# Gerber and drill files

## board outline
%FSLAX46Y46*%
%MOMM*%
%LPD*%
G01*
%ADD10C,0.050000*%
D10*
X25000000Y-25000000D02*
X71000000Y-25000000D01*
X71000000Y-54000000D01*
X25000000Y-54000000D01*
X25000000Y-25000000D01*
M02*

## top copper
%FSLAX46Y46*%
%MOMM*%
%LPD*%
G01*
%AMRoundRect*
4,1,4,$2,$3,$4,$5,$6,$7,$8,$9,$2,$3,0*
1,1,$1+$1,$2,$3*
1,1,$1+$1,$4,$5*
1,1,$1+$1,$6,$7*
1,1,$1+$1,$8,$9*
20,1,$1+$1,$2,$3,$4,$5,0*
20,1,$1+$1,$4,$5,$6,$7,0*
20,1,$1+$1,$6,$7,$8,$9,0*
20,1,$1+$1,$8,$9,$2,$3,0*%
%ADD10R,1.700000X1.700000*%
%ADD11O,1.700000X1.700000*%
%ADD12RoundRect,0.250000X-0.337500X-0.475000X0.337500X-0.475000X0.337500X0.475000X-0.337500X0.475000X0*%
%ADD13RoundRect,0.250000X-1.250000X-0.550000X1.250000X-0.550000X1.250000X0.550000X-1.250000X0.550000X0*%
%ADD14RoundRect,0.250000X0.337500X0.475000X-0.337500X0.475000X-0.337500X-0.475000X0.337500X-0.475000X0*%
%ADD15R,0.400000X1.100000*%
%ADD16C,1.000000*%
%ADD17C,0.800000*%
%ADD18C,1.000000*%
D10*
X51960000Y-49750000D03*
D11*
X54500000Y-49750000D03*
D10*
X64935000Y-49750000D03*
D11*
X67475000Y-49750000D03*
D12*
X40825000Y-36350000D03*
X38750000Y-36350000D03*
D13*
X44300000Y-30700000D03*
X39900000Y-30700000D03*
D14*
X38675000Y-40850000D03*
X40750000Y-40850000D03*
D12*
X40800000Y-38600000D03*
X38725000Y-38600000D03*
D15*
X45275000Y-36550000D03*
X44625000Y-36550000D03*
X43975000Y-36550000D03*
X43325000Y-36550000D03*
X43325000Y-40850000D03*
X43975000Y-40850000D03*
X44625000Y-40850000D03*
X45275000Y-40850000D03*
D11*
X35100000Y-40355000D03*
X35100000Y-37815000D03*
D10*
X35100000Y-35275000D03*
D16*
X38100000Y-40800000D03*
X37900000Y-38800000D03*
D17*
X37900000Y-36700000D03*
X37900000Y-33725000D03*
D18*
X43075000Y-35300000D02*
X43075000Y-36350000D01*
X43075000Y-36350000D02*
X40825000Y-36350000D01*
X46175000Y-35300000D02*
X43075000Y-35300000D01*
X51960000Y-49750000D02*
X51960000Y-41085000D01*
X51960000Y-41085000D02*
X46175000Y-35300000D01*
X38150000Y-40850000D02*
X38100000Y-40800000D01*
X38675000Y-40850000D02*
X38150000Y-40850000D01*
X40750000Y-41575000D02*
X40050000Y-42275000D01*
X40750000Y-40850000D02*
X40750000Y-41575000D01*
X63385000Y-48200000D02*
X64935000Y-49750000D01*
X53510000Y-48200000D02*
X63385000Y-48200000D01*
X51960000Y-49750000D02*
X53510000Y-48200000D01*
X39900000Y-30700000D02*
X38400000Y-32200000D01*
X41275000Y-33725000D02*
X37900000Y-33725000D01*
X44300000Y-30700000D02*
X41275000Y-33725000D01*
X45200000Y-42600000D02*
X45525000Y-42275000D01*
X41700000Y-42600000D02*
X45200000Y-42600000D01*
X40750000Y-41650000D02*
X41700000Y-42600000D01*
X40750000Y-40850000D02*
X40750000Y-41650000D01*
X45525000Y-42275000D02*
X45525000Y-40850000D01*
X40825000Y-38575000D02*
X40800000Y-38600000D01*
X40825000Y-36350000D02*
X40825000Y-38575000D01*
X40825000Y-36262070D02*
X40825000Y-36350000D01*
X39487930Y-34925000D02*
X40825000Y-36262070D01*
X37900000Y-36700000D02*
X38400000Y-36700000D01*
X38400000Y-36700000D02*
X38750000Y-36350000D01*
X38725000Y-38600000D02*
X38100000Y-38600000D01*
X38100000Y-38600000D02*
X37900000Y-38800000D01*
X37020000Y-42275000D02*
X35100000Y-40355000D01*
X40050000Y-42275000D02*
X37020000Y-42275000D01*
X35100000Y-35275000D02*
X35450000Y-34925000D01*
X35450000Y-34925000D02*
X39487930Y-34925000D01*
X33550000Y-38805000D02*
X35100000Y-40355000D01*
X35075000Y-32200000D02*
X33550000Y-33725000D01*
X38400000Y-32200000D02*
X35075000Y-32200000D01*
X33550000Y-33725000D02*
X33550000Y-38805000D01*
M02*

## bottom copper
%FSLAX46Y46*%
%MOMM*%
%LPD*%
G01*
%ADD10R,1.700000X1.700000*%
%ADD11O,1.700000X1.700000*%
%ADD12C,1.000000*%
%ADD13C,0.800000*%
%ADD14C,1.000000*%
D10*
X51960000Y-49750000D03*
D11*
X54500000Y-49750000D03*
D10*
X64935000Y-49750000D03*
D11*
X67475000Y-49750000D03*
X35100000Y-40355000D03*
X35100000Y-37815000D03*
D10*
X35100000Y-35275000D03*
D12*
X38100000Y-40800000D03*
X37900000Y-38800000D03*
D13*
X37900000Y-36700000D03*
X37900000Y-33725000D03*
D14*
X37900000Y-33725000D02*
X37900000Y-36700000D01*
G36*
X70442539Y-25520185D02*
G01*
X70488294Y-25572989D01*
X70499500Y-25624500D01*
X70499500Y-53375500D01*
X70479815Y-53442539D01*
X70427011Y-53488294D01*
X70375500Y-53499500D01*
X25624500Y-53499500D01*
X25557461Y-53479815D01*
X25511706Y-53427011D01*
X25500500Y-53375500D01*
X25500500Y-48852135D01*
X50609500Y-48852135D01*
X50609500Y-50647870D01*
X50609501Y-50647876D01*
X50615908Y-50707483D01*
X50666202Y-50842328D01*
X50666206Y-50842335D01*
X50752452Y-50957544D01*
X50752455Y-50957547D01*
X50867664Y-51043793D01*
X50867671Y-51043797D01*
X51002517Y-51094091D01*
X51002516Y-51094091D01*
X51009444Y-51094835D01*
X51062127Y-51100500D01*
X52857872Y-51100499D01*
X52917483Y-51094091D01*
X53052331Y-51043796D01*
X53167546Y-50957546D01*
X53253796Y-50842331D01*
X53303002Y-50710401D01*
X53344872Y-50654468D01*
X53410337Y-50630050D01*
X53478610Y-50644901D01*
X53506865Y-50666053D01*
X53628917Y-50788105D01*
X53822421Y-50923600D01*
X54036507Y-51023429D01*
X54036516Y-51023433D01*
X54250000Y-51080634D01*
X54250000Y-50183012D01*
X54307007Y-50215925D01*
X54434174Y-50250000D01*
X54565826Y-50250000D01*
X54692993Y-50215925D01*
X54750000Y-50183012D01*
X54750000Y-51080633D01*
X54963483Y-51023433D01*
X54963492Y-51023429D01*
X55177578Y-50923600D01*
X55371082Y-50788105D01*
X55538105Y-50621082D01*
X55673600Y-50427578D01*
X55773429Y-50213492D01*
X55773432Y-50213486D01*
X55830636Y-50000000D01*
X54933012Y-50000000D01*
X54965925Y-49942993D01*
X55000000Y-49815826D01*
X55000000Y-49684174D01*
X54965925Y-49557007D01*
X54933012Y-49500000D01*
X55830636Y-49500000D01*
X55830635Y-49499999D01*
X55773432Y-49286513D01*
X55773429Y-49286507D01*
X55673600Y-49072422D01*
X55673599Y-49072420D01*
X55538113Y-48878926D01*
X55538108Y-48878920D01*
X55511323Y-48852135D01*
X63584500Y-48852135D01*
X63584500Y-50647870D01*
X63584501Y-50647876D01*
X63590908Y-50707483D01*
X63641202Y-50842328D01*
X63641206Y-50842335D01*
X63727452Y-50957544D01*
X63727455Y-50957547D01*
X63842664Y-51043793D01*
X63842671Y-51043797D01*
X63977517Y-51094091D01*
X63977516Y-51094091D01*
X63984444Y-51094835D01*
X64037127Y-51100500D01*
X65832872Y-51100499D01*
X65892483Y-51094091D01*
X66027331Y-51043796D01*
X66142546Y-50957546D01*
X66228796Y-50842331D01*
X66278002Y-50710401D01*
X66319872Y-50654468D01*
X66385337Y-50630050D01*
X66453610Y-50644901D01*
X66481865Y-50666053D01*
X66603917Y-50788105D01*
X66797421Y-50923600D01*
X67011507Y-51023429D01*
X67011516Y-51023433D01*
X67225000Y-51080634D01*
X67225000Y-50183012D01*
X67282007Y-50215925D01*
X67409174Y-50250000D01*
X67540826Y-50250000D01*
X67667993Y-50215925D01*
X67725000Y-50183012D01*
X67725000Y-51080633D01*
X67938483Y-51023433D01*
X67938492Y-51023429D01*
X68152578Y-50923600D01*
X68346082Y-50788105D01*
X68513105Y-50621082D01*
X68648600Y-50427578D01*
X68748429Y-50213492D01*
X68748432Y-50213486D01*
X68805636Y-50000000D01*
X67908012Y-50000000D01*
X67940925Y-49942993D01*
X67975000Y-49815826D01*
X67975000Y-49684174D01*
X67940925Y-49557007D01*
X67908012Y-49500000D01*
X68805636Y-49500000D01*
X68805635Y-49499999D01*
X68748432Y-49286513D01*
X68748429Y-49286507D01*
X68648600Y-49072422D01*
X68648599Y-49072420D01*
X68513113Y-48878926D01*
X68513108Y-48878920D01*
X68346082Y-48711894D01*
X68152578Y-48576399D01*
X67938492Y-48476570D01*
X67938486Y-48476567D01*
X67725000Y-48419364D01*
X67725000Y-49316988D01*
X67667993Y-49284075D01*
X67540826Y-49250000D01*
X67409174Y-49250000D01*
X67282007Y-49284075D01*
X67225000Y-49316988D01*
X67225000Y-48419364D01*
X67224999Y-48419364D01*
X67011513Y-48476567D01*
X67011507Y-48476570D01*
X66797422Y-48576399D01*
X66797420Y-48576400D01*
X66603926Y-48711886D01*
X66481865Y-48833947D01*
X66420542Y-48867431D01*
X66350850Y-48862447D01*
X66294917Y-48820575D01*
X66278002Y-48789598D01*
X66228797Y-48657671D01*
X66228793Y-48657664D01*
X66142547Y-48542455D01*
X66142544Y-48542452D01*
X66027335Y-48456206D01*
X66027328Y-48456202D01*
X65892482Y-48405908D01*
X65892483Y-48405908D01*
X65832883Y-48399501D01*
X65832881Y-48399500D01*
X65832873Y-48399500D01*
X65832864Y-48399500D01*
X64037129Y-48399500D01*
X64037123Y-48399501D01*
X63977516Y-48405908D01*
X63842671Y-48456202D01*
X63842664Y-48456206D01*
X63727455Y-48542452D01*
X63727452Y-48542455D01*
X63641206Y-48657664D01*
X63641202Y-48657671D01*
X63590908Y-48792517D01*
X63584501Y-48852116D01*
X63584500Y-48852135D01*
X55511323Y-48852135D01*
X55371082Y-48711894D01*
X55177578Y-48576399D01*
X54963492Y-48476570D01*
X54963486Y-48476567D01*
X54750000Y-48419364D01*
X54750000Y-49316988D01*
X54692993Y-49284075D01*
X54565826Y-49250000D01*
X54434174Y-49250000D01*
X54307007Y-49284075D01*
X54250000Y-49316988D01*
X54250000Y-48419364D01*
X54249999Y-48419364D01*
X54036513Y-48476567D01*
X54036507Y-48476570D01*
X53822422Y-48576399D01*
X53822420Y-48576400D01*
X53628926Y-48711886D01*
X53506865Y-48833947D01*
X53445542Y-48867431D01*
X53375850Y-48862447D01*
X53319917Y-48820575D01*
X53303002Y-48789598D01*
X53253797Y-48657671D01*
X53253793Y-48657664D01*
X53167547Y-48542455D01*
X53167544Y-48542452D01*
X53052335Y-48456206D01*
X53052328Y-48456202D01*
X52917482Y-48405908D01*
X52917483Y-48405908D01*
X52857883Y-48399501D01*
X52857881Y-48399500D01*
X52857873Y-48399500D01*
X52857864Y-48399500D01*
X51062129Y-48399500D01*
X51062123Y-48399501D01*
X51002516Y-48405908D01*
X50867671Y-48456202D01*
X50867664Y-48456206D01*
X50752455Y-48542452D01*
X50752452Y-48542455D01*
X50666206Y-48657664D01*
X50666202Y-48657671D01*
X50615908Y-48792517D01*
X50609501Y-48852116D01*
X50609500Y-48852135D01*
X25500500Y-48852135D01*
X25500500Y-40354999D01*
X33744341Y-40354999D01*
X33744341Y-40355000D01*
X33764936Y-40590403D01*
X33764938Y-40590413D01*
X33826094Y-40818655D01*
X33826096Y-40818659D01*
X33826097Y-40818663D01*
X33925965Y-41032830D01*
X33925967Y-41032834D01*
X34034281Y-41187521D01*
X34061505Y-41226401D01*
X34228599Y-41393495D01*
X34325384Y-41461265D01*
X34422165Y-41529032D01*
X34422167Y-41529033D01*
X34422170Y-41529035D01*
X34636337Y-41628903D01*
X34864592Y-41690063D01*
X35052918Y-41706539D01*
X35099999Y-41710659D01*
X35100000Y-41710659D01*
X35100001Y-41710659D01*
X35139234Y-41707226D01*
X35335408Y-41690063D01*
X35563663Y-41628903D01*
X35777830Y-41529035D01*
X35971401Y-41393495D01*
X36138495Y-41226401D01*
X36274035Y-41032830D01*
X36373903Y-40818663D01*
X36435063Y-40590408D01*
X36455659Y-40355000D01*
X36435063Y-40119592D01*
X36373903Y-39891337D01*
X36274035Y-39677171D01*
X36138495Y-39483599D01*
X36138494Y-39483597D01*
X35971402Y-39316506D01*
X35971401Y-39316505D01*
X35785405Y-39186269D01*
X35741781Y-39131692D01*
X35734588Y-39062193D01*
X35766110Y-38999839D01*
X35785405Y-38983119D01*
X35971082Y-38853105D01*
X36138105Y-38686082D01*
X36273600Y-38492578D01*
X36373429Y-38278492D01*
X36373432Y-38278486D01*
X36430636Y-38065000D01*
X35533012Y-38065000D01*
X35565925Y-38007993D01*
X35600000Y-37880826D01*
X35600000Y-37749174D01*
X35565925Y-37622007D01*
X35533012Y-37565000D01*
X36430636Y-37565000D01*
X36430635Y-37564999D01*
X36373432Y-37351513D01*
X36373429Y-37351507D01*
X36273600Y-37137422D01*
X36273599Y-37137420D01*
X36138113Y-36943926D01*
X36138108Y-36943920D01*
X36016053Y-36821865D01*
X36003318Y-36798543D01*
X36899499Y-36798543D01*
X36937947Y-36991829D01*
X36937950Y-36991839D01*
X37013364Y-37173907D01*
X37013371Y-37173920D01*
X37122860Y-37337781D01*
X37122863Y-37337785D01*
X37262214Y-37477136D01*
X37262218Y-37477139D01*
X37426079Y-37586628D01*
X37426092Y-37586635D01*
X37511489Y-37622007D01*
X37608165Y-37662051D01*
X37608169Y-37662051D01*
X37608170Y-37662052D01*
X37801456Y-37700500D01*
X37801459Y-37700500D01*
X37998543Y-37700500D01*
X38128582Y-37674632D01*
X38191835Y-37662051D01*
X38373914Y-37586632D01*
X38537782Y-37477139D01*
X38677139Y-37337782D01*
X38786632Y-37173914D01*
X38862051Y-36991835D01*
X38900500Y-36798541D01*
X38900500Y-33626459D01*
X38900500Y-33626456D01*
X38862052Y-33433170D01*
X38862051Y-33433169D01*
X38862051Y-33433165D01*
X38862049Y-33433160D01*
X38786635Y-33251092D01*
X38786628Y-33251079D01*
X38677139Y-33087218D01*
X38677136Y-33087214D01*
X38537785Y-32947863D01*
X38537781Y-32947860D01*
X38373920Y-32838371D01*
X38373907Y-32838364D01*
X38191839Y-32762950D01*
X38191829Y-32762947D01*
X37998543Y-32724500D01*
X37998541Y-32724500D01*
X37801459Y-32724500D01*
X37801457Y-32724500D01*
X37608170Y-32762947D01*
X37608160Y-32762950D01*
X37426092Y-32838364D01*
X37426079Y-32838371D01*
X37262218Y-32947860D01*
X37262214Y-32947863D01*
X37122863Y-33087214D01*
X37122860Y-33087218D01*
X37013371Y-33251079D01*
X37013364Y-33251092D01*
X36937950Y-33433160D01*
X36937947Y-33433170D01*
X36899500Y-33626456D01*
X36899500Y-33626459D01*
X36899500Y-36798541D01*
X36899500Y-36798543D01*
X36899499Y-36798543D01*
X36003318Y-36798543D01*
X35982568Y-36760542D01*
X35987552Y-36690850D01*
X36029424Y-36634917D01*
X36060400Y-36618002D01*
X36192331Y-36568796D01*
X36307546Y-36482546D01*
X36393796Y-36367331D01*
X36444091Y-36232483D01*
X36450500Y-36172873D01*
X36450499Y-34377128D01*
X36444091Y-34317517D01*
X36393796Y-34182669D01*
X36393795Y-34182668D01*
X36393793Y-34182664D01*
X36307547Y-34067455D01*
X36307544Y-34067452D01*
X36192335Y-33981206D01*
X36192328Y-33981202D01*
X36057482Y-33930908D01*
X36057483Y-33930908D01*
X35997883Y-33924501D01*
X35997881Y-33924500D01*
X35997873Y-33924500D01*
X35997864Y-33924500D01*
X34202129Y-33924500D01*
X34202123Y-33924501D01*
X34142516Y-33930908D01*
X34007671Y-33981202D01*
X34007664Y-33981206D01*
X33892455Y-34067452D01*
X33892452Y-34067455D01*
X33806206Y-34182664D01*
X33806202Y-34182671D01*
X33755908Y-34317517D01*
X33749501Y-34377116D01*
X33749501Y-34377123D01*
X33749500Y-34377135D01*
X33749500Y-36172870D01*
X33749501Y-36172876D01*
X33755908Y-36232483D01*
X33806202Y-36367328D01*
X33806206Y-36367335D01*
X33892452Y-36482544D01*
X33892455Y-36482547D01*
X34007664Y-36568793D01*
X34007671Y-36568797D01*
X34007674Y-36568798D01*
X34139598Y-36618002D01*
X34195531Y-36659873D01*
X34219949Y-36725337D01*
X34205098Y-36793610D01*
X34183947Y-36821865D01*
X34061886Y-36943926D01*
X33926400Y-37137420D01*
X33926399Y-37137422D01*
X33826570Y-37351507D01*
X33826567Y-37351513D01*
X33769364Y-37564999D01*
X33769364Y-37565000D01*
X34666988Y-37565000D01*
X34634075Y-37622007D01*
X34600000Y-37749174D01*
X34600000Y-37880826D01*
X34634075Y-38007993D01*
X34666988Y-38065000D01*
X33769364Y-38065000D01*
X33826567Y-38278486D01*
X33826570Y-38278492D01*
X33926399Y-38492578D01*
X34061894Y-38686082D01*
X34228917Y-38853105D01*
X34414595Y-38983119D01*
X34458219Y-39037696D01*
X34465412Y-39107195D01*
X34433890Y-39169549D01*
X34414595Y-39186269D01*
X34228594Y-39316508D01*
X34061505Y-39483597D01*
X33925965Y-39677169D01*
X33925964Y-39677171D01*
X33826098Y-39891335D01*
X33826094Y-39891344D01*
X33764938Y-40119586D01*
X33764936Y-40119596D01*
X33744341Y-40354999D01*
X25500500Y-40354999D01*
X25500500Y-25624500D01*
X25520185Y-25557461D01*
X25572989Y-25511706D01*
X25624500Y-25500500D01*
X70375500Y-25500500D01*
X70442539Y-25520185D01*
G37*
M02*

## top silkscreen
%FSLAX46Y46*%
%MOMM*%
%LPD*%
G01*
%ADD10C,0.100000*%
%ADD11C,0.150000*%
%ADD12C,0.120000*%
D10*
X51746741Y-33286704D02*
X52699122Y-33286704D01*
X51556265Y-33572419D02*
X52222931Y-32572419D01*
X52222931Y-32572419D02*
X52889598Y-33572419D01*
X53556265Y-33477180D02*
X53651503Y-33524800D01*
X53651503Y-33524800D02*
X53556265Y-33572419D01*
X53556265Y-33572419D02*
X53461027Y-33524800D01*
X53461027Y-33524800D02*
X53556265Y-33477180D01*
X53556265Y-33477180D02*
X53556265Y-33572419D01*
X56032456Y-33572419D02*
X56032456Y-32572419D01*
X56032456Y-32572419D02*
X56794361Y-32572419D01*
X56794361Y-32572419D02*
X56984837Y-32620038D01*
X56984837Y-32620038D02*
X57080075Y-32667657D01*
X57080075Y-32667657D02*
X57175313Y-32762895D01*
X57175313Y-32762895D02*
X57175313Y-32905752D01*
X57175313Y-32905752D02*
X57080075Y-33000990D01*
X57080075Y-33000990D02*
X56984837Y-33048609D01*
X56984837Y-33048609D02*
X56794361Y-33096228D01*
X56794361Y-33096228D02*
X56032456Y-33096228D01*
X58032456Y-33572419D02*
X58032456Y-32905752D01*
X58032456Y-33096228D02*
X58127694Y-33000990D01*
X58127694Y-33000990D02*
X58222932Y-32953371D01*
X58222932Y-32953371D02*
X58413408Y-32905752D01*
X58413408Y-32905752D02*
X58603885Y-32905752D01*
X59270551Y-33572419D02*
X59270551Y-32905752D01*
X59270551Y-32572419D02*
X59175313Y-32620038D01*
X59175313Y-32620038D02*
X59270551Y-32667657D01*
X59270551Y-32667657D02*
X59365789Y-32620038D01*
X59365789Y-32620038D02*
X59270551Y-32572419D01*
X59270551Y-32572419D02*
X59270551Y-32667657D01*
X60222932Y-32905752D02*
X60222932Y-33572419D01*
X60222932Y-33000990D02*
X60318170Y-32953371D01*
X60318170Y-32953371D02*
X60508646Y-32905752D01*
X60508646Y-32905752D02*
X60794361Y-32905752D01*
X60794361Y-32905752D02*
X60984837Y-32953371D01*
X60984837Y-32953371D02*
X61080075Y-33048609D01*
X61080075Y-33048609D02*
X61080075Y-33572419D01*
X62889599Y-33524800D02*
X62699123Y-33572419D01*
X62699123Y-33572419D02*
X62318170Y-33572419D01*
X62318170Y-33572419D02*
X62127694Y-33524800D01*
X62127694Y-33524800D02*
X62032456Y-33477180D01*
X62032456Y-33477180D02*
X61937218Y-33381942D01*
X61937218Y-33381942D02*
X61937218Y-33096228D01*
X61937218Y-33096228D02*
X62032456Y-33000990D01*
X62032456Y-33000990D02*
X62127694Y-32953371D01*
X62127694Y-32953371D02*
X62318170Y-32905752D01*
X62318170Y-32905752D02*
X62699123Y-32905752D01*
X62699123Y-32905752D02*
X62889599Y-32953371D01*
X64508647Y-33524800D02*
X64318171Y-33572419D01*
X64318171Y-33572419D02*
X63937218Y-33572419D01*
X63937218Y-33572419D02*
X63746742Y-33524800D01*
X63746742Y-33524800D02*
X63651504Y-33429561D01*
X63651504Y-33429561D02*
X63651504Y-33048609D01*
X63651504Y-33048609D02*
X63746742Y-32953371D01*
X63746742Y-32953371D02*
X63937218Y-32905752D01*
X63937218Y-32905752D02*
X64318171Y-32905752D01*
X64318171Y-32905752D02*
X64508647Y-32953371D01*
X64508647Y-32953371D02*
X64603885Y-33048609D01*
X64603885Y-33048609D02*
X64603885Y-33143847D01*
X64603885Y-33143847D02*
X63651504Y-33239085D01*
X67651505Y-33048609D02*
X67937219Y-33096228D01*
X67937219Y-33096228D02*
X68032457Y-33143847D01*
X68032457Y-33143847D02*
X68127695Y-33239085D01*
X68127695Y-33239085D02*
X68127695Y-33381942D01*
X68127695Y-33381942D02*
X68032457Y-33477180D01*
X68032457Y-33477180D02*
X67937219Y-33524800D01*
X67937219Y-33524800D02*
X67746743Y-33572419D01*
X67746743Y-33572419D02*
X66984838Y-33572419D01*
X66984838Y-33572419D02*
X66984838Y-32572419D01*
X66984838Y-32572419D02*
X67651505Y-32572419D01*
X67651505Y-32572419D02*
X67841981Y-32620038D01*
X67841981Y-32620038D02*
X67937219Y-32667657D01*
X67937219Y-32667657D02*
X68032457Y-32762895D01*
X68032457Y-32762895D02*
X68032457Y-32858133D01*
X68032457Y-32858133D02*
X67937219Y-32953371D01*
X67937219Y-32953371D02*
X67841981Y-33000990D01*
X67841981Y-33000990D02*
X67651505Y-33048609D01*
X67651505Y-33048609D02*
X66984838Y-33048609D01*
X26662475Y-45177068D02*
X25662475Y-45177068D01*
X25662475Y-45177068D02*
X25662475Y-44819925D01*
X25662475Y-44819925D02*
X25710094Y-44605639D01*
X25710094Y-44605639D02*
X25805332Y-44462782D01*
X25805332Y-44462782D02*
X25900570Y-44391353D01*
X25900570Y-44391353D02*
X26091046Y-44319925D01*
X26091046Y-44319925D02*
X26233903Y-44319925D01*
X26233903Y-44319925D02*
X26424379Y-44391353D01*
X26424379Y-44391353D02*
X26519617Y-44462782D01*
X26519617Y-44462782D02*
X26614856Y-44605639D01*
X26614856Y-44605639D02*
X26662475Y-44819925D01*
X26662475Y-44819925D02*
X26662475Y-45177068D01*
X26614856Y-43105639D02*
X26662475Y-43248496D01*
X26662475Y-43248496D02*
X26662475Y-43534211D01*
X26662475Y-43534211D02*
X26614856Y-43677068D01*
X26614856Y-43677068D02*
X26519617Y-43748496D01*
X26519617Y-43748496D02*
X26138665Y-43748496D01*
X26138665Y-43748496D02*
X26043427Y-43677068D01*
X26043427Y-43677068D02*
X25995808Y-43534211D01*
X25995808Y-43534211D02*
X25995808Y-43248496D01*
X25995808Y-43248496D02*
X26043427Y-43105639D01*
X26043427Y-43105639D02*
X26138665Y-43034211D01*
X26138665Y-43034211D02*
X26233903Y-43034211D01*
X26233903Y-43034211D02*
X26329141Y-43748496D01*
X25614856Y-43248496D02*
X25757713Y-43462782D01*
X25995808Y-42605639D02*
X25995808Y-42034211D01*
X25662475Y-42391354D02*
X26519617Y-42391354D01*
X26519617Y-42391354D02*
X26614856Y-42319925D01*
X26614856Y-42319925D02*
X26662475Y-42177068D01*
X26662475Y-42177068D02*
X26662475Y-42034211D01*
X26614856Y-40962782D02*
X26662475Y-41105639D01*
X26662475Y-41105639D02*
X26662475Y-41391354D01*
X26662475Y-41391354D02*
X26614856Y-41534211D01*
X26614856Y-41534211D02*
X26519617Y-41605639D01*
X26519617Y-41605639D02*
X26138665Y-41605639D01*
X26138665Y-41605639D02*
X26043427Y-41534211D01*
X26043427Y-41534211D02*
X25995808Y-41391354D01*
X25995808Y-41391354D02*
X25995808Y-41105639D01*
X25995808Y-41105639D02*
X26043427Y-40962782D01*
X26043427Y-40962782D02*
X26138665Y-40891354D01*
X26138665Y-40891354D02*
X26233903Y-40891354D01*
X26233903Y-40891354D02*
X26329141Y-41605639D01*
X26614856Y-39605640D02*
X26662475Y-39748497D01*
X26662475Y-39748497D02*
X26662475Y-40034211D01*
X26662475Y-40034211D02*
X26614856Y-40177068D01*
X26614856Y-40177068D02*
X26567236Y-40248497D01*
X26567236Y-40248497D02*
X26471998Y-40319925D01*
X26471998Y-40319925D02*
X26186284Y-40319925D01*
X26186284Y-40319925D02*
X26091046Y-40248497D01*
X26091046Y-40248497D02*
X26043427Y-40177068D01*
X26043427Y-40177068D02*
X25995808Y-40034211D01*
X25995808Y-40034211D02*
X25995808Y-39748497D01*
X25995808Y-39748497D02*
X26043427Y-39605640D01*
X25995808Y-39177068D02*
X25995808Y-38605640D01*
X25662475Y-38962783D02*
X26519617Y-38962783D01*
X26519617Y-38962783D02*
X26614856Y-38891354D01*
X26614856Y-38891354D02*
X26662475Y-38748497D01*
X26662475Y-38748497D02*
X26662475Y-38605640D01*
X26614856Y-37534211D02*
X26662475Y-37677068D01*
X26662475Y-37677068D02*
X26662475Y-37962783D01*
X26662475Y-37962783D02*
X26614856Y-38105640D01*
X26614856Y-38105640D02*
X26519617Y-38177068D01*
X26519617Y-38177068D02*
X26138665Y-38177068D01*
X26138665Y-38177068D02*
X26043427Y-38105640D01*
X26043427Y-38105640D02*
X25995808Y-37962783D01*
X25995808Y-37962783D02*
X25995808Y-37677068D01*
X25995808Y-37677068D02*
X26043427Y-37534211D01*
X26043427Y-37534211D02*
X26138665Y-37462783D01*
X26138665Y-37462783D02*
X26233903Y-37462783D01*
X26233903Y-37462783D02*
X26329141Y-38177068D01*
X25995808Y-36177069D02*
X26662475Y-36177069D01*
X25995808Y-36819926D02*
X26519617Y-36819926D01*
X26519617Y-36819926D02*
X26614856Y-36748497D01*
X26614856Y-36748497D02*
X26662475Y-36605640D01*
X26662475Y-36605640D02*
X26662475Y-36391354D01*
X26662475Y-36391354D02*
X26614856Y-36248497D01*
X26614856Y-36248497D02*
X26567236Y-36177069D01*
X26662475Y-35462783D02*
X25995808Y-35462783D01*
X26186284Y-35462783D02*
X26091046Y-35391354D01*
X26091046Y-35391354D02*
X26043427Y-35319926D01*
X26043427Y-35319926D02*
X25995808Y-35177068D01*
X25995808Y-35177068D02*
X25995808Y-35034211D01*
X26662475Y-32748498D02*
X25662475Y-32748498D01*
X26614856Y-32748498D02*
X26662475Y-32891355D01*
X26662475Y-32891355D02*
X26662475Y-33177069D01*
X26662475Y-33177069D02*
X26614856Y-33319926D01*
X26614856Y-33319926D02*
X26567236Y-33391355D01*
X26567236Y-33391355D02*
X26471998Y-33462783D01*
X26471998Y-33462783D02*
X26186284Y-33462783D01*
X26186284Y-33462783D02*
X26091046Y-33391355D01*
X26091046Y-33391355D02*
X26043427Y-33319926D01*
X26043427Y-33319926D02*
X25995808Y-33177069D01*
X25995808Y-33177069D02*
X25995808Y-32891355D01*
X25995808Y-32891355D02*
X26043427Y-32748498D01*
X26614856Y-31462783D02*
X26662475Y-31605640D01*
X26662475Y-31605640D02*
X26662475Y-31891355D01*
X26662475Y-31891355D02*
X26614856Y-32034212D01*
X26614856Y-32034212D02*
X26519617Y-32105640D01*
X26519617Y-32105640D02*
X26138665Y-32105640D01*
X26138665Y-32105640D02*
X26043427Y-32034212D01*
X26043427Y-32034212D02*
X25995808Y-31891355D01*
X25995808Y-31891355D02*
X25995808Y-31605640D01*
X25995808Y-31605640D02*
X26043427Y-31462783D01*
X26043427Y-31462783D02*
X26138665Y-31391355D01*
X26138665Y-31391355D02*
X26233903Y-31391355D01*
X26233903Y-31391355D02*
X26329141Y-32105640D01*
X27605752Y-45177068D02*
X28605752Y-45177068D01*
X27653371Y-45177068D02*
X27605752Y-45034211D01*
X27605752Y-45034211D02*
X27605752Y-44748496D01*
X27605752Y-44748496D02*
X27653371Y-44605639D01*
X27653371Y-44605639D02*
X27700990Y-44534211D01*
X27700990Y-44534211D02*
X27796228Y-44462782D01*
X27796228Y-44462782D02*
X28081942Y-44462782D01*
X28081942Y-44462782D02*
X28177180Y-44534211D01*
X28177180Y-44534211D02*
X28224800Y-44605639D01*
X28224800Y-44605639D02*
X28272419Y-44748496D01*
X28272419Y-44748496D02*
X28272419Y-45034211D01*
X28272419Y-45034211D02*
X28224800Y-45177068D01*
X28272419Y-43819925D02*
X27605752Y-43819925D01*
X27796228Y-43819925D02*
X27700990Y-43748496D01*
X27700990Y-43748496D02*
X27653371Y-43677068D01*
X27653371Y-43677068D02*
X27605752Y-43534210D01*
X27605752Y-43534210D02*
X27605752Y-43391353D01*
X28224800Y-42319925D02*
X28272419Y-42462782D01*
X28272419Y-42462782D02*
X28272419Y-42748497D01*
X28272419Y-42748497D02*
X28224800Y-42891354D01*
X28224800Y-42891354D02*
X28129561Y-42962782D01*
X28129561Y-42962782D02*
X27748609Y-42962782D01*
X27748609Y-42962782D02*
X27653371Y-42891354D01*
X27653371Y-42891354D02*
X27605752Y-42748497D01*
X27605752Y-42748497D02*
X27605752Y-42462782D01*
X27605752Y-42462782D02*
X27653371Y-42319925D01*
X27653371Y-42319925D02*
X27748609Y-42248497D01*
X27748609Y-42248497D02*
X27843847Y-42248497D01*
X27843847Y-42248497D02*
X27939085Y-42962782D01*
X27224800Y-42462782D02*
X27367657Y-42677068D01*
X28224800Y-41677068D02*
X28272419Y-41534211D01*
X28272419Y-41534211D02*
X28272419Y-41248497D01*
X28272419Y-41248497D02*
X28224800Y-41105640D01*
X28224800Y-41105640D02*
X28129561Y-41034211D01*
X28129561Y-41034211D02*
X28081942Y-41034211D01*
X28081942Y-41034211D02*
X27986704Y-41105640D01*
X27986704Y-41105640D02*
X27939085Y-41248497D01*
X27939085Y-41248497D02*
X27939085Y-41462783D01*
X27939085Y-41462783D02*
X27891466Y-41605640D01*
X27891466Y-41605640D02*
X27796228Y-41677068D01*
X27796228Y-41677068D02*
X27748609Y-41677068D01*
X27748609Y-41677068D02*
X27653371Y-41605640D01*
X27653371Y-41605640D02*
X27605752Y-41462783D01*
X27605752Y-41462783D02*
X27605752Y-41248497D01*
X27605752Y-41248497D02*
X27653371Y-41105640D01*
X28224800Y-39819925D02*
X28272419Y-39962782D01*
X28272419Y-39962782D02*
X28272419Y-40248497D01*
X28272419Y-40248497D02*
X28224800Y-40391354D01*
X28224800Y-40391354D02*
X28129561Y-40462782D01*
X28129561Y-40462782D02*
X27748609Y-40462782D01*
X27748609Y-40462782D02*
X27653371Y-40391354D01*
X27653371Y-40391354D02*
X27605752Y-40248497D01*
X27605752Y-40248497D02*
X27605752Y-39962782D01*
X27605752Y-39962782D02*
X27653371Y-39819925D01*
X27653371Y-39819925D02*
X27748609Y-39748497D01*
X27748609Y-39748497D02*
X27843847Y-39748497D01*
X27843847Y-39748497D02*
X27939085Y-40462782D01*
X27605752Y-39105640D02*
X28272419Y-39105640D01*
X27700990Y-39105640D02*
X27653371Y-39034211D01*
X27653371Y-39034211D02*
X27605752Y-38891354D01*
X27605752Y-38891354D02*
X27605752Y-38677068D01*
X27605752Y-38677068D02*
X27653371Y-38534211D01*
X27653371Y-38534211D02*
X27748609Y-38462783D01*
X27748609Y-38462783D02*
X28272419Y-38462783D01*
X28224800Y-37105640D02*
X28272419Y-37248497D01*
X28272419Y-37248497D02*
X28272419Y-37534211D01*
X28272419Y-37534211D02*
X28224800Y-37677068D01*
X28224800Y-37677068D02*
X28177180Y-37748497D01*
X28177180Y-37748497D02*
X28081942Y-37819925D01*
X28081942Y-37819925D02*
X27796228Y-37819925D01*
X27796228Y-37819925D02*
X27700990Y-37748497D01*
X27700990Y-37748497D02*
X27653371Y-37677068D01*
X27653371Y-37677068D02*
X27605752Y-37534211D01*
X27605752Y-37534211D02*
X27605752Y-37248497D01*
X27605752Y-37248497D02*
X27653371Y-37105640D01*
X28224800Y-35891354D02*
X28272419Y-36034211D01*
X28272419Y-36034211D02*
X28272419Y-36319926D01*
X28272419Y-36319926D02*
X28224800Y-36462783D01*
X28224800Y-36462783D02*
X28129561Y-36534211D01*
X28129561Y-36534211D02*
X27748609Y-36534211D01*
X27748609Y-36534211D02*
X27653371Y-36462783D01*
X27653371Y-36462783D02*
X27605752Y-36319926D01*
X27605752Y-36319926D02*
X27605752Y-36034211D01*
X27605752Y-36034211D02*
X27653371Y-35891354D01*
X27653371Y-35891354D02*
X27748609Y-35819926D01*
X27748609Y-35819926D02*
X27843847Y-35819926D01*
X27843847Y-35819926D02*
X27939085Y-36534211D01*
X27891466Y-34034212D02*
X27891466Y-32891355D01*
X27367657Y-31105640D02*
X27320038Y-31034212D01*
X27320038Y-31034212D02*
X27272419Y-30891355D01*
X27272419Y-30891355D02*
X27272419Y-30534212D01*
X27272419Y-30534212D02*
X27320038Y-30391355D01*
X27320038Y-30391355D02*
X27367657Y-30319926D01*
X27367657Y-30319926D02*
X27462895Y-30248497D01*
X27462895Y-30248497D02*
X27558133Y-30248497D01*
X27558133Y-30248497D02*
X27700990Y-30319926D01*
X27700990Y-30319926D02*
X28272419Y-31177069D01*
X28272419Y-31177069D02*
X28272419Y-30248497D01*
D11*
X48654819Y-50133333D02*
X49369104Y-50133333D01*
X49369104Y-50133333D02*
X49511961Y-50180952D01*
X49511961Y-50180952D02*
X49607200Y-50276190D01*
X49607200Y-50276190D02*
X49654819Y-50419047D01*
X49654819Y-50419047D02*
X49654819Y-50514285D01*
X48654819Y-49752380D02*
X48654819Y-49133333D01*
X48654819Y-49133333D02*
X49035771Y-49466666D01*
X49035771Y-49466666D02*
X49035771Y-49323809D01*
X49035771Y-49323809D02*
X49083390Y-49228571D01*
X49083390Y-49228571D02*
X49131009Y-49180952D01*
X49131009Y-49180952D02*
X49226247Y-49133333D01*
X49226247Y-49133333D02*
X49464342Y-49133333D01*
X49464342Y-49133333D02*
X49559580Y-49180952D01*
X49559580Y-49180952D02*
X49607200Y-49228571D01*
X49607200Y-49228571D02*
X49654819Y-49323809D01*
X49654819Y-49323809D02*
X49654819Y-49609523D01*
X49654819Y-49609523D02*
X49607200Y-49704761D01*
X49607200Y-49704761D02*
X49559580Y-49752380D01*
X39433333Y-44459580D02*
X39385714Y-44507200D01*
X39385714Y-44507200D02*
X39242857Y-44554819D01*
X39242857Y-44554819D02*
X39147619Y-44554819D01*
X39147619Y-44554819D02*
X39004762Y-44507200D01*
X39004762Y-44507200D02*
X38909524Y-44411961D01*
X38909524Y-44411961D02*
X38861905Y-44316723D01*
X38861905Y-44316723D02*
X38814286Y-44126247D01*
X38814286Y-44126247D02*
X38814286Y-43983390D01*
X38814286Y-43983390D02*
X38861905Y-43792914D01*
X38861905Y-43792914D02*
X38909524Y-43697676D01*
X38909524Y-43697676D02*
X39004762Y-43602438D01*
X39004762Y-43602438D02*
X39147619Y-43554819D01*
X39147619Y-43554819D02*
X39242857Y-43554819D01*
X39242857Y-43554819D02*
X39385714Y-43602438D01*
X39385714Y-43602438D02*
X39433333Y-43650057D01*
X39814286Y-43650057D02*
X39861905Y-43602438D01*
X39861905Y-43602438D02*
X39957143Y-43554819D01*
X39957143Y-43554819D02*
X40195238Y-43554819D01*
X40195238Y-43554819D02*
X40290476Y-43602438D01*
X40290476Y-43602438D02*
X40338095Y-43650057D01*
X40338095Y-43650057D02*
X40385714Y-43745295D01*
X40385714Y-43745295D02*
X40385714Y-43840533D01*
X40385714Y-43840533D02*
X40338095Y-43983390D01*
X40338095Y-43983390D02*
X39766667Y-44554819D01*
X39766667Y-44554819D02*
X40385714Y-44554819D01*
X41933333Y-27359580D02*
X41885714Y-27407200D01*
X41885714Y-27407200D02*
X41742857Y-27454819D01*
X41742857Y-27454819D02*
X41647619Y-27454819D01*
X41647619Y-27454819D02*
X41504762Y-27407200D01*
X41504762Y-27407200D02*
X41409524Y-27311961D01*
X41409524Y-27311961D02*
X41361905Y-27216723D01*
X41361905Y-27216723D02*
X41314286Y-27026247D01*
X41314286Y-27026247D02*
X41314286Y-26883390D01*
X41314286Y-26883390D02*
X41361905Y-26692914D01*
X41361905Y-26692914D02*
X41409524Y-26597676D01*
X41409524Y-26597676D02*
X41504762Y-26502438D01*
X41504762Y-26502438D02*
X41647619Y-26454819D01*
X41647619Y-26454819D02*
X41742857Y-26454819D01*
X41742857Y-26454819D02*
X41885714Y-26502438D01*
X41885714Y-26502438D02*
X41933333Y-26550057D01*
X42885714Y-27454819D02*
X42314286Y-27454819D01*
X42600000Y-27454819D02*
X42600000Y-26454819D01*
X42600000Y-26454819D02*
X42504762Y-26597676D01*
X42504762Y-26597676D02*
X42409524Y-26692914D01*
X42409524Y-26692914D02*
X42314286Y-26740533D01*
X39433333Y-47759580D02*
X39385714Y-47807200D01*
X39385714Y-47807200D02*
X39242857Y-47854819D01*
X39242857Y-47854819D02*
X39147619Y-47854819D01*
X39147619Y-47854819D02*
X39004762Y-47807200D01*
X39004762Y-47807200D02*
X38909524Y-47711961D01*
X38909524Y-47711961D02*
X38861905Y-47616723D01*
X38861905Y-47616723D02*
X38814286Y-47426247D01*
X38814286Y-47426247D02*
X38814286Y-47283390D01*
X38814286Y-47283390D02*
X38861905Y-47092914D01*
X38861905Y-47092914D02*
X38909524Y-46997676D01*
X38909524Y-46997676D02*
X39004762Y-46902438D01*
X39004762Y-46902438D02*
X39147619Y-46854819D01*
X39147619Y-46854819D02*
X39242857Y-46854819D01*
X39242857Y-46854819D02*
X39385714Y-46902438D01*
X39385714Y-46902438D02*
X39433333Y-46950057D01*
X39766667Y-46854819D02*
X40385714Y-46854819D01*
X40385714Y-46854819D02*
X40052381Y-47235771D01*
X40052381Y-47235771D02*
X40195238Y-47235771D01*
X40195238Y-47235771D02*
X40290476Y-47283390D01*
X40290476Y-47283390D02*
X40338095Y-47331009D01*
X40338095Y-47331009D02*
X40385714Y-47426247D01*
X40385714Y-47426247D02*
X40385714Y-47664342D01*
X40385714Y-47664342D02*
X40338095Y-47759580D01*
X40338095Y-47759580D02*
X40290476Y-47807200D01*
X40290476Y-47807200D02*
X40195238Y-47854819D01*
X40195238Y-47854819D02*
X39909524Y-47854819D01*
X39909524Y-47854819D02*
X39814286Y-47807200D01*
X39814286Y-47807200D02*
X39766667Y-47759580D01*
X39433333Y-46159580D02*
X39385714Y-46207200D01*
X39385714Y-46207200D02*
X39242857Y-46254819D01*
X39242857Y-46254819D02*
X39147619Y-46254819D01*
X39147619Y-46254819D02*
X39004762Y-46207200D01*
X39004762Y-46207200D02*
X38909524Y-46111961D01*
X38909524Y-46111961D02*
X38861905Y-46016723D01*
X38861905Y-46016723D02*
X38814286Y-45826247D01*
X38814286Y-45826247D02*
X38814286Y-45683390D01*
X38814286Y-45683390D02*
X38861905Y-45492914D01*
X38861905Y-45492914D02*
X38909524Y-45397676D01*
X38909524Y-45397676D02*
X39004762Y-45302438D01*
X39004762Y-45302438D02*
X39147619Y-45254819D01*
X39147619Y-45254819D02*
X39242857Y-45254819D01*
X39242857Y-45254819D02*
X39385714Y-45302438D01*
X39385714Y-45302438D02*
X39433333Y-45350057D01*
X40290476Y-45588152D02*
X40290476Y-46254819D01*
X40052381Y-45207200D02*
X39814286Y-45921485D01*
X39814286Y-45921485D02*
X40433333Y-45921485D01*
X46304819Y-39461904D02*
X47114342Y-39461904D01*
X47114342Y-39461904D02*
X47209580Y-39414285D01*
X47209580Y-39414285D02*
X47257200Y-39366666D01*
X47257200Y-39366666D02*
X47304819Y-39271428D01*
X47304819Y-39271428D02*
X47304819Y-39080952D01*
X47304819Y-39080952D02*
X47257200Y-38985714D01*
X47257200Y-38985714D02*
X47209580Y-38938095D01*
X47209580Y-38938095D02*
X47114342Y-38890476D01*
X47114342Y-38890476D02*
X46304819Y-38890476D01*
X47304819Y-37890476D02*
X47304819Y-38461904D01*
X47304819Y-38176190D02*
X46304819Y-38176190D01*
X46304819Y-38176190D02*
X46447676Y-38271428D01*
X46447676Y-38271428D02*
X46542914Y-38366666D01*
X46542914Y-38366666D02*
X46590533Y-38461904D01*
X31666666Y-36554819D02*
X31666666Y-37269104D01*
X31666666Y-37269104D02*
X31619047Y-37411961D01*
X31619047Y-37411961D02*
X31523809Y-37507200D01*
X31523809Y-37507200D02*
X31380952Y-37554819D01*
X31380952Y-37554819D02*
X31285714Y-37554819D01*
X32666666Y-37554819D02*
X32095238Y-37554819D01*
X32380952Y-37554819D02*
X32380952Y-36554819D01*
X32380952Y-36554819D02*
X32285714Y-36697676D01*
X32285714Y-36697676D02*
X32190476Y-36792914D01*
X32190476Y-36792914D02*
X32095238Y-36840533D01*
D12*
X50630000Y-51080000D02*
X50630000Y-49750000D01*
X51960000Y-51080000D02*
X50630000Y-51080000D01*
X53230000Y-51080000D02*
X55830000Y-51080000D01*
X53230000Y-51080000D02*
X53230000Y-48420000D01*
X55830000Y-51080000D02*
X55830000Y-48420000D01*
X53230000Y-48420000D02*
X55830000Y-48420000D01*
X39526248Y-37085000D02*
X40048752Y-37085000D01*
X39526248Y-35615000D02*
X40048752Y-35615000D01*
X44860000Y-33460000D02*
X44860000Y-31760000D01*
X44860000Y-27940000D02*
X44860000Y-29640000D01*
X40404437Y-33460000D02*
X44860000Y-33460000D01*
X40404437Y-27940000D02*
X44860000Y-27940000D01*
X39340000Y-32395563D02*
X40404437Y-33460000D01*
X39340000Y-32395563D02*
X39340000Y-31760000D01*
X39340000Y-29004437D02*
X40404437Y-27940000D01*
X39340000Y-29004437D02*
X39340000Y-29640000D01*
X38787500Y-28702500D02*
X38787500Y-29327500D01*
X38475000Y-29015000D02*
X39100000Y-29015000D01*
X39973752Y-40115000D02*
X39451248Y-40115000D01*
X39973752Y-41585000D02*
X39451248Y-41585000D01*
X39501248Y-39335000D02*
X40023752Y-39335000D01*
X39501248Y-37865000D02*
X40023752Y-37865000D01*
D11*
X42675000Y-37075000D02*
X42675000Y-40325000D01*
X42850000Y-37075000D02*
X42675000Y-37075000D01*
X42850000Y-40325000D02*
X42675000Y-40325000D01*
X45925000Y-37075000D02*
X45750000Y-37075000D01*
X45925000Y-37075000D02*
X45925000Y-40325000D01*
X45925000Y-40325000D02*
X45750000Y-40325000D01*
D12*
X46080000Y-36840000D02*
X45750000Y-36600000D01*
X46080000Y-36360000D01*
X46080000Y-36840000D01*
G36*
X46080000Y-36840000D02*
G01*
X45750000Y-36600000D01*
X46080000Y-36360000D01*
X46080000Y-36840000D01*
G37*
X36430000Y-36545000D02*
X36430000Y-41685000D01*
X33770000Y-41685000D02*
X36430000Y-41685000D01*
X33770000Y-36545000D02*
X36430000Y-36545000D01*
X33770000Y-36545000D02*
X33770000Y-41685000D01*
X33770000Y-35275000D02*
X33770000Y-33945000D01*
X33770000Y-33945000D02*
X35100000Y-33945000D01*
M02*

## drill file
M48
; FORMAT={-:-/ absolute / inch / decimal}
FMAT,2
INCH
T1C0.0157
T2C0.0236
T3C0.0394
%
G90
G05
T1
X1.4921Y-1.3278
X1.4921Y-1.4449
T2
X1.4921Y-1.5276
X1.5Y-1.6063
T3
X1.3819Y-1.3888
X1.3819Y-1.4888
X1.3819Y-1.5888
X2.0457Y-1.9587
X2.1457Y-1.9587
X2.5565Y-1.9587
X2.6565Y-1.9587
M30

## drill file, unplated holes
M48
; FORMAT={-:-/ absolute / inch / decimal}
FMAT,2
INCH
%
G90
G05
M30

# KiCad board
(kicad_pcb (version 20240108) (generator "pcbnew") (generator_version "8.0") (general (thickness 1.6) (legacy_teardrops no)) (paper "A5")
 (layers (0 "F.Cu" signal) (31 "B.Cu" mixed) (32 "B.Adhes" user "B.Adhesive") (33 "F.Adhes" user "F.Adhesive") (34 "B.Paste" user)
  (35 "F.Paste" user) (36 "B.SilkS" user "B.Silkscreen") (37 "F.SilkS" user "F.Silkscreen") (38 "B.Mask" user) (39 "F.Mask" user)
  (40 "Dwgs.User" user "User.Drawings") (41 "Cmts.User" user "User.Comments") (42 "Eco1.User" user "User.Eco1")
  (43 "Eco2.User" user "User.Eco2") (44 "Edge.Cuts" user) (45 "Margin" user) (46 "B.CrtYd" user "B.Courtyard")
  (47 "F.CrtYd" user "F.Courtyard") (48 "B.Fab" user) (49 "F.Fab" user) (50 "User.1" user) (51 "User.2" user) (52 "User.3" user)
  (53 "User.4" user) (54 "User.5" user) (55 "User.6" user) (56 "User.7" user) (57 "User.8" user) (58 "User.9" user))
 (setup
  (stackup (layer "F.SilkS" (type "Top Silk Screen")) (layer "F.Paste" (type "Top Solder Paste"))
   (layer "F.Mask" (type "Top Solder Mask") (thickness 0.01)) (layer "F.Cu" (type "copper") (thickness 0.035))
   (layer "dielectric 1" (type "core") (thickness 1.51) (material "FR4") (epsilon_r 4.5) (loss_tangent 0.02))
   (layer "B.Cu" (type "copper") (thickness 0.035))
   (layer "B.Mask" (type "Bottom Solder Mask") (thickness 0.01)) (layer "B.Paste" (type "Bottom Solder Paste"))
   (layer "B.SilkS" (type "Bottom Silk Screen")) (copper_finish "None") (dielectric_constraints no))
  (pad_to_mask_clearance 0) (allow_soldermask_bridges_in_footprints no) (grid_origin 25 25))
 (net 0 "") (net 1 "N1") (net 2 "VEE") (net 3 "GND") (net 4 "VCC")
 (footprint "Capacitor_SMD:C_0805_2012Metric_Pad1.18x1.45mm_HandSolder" (layer "F.Cu") (at 39.7875 36.35)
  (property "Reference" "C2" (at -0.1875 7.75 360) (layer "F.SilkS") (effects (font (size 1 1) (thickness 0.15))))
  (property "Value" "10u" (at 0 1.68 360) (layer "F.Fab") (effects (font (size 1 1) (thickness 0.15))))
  (fp_line (start -0.261252 -0.735) (end 0.261252 -0.735) (stroke (width 0.12) (type solid)) (layer "F.SilkS"))
  (fp_line (start -0.261252 0.735) (end 0.261252 0.735) (stroke (width 0.12) (type solid)) (layer "F.SilkS"))
  (pad "1" smd roundrect (at -1.0375 0) (size 1.175 1.45) (layers "F.Cu" "F.Paste" "F.Mask") (roundrect_rratio 0.212766) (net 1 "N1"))
  (pad "2" smd roundrect (at 1.0375 0) (size 1.175 1.45) (layers "F.Cu" "F.Paste" "F.Mask") (roundrect_rratio 0.212766) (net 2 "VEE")))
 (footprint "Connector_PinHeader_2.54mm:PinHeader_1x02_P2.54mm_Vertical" (layer "F.Cu") (at 51.96 49.75 90)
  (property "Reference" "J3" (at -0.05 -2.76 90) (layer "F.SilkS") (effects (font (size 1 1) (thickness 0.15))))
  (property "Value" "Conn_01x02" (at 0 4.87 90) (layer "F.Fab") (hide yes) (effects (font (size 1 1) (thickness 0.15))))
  (fp_line (start -1.33 -1.33) (end 0 -1.33) (stroke (width 0.12) (type solid)) (layer "F.SilkS"))
  (fp_line (start -1.33 0) (end -1.33 -1.33) (stroke (width 0.12) (type solid)) (layer "F.SilkS"))
  (fp_line (start 1.33 1.27) (end 1.33 3.87) (stroke (width 0.12) (type solid)) (layer "F.SilkS"))
  (fp_line (start -1.33 1.27) (end 1.33 1.27) (stroke (width 0.12) (type solid)) (layer "F.SilkS"))
  (fp_line (start -1.33 1.27) (end -1.33 3.87) (stroke (width 0.12) (type solid)) (layer "F.SilkS"))
  (fp_line (start -1.33 3.87) (end 1.33 3.87) (stroke (width 0.12) (type solid)) (layer "F.SilkS"))
  (pad "1" thru_hole rect (at 0 0 90) (size 1.7 1.7) (drill 1) (layers "*.Cu" "*.Mask") (remove_unused_layers no) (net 2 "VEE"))
  (pad "2" thru_hole oval (at 0 2.54 90) (size 1.7 1.7) (drill 1) (layers "*.Cu" "*.Mask") (remove_unused_layers no) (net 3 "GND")))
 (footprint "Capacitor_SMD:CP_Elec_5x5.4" (layer "F.Cu") (at 42.1 30.7)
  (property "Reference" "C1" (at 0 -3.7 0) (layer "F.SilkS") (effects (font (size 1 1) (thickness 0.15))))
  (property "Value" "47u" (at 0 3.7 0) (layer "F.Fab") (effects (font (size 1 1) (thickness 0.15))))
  (fp_line (start -3.625 -1.685) (end -3 -1.685) (stroke (width 0.12) (type solid)) (layer "F.SilkS"))
  (fp_line (start -3.3125 -1.9975) (end -3.3125 -1.3725) (stroke (width 0.12) (type solid)) (layer "F.SilkS"))
  (fp_line (start -2.76 -1.695563) (end -2.76 -1.06) (stroke (width 0.12) (type solid)) (layer "F.SilkS"))
  (fp_line (start -2.76 -1.695563) (end -1.695563 -2.76) (stroke (width 0.12) (type solid)) (layer "F.SilkS"))
  (fp_line (start -2.76 1.695563) (end -2.76 1.06) (stroke (width 0.12) (type solid)) (layer "F.SilkS"))
  (fp_line (start -2.76 1.695563) (end -1.695563 2.76) (stroke (width 0.12) (type solid)) (layer "F.SilkS"))
  (fp_line (start -1.695563 -2.76) (end 2.76 -2.76) (stroke (width 0.12) (type solid)) (layer "F.SilkS"))
  (fp_line (start -1.695563 2.76) (end 2.76 2.76) (stroke (width 0.12) (type solid)) (layer "F.SilkS"))
  (fp_line (start 2.76 -2.76) (end 2.76 -1.06) (stroke (width 0.12) (type solid)) (layer "F.SilkS"))
  (fp_line (start 2.76 2.76) (end 2.76 1.06) (stroke (width 0.12) (type solid)) (layer "F.SilkS"))
  (pad "1" smd roundrect (at -2.2 0) (size 3 1.6) (layers "F.Cu" "F.Paste" "F.Mask") (roundrect_rratio 0.15625) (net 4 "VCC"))
  (pad "2" smd roundrect (at 2.2 0) (size 3 1.6) (layers "F.Cu" "F.Paste" "F.Mask") (roundrect_rratio 0.15625) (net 1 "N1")))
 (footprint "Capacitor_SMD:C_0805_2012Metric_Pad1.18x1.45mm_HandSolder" (layer "F.Cu") (at 39.7125 40.85 180)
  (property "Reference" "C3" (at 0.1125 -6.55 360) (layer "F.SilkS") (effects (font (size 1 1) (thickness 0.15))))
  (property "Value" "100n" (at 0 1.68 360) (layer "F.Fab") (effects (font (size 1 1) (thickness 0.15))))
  (fp_line (start -0.261252 0.735) (end 0.261252 0.735) (stroke (width 0.12) (type solid)) (layer "F.SilkS"))
  (fp_line (start -0.261252 -0.735) (end 0.261252 -0.735) (stroke (width 0.12) (type solid)) (layer "F.SilkS"))
  (pad "1" smd roundrect (at -1.0375 0 180) (size 1.175 1.45) (layers "F.Cu" "F.Paste" "F.Mask") (roundrect_rratio 0.212766) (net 4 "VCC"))
  (pad "2" smd roundrect (at 1.0375 0 180) (size 1.175 1.45) (layers "F.Cu" "F.Paste" "F.Mask") (roundrect_rratio 0.212766) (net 3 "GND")))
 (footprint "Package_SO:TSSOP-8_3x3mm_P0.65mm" (layer "F.Cu") (at 44.3 38.7 -90)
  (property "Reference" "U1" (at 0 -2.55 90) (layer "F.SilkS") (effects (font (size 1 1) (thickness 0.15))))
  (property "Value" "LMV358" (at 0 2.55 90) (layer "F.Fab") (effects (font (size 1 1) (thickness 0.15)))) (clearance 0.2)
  (fp_line (start -1.625 1.625) (end 1.625 1.625) (stroke (width 0.15) (type solid)) (layer "F.SilkS"))
  (fp_line (start -1.625 1.45) (end -1.625 1.625) (stroke (width 0.15) (type solid)) (layer "F.SilkS"))
  (fp_line (start 1.625 1.45) (end 1.625 1.625) (stroke (width 0.15) (type solid)) (layer "F.SilkS"))
  (fp_line (start -1.625 -1.625) (end -1.625 -1.45) (stroke (width 0.15) (type solid)) (layer "F.SilkS"))
  (fp_line (start -1.625 -1.625) (end 1.625 -1.625) (stroke (width 0.15) (type solid)) (layer "F.SilkS"))
  (fp_line (start 1.625 -1.625) (end 1.625 -1.45) (stroke (width 0.15) (type solid)) (layer "F.SilkS"))
  (fp_poly
   (pts (xy -2.1 -1.45) (xy -2.34 -1.78) (xy -1.86 -1.78) (xy -2.1 -1.45)) (stroke (width 0.12) (type solid)) (fill solid) (layer "F.SilkS"))
  (pad "1" smd rect (at -2.15 -0.975 270) (size 1.1 0.4) (layers "F.Cu" "F.Paste" "F.Mask"))
  (pad "2" smd rect (at -2.15 -0.325 270) (size 1.1 0.4) (layers "F.Cu" "F.Paste" "F.Mask"))
  (pad "3" smd rect (at -2.15 0.325 270) (size 1.1 0.4) (layers "F.Cu" "F.Paste" "F.Mask"))
  (pad "4" smd rect (at -2.15 0.975 270) (size 1.1 0.4) (layers "F.Cu" "F.Paste" "F.Mask") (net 2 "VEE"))
  (pad "5" smd rect (at 2.15 0.975 270) (size 1.1 0.4) (layers "F.Cu" "F.Paste" "F.Mask"))
  (pad "6" smd rect (at 2.15 0.325 270) (size 1.1 0.4) (layers "F.Cu" "F.Paste" "F.Mask"))
  (pad "7" smd rect (at 2.15 -0.325 270) (size 1.1 0.4) (layers "F.Cu" "F.Paste" "F.Mask"))
  (pad "8" smd rect (at 2.15 -0.975 270) (size 1.1 0.4) (layers "F.Cu" "F.Paste" "F.Mask") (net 4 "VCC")))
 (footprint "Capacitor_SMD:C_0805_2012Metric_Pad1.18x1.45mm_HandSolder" (layer "F.Cu") (at 39.7625 38.6)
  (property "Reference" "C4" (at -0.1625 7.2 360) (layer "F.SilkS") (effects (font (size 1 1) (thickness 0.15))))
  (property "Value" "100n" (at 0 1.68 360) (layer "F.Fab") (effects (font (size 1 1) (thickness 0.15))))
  (fp_line (start -0.261252 -0.735) (end 0.261252 -0.735) (stroke (width 0.12) (type solid)) (layer "F.SilkS"))
  (fp_line (start -0.261252 0.735) (end 0.261252 0.735) (stroke (width 0.12) (type solid)) (layer "F.SilkS"))
  (pad "1" smd roundrect (at -1.0375 0) (size 1.175 1.45) (layers "F.Cu" "F.Paste" "F.Mask") (roundrect_rratio 0.212766) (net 3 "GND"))
  (pad "2" smd roundrect (at 1.0375 0) (size 1.175 1.45) (layers "F.Cu" "F.Paste" "F.Mask") (roundrect_rratio 0.212766) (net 2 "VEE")))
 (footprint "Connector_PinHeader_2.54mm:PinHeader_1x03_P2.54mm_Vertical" (layer "F.Cu") (at 35.1 35.275)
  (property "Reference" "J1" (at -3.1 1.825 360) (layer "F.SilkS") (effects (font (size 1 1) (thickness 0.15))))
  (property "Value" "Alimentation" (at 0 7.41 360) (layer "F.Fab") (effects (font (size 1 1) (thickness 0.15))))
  (fp_line (start -1.33 -1.33) (end 0 -1.33) (stroke (width 0.12) (type solid)) (layer "F.SilkS"))
  (fp_line (start -1.33 0) (end -1.33 -1.33) (stroke (width 0.12) (type solid)) (layer "F.SilkS"))
  (fp_line (start -1.33 1.27) (end -1.33 6.41) (stroke (width 0.12) (type solid)) (layer "F.SilkS"))
  (fp_line (start -1.33 1.27) (end 1.33 1.27) (stroke (width 0.12) (type solid)) (layer "F.SilkS"))
  (fp_line (start -1.33 6.41) (end 1.33 6.41) (stroke (width 0.12) (type solid)) (layer "F.SilkS"))
  (fp_line (start 1.33 1.27) (end 1.33 6.41) (stroke (width 0.12) (type solid)) (layer "F.SilkS"))
  (pad "1" thru_hole rect (at 0 0) (size 1.7 1.7) (drill 1) (layers "*.Cu" "*.Mask") (remove_unused_layers no) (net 2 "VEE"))
  (pad "2" thru_hole oval (at 0 2.54) (size 1.7 1.7) (drill 1) (layers "*.Cu" "*.Mask") (remove_unused_layers no) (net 3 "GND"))
  (pad "3" thru_hole oval (at 0 5.08) (size 1.7 1.7) (drill 1) (layers "*.Cu" "*.Mask") (remove_unused_layers no) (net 4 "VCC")))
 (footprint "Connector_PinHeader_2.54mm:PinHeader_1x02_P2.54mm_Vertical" (layer "B.Cu") (at 64.935 49.75 -90)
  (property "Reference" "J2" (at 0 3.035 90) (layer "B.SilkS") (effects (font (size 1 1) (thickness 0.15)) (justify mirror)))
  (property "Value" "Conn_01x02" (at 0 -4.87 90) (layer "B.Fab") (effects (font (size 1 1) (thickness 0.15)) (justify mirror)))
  (pad "1" thru_hole rect (at 0 0 270) (size 1.7 1.7) (drill 1) (layers "*.Cu" "*.Mask") (remove_unused_layers no) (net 2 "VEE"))
  (pad "2" thru_hole oval (at 0 -2.54 270) (size 1.7 1.7) (drill 1) (layers "*.Cu" "*.Mask") (remove_unused_layers no) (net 3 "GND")))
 (gr_rect (start 25 25) (end 71 54) (stroke (width 0.05) (type default)) (fill none) (layer "Edge.Cuts"))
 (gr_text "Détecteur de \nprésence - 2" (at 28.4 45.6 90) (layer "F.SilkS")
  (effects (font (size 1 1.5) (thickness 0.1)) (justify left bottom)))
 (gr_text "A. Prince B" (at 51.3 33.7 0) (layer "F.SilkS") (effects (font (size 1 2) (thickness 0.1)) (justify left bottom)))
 (segment (start 37.02 42.275) (end 35.1 40.355) (width 1) (layer "F.Cu") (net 4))
 (segment (start 40.05 42.275) (end 37.02 42.275) (width 1) (layer "F.Cu") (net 4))
 (segment (start 45.2 42.6) (end 45.525 42.275) (width 1) (layer "F.Cu") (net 4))
 (segment (start 33.55 33.725) (end 33.55 38.805) (width 1) (layer "F.Cu") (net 4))
 (segment (start 38.4 32.2) (end 35.075 32.2) (width 1) (layer "F.Cu") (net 4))
 (segment (start 35.075 32.2) (end 33.55 33.725) (width 1) (layer "F.Cu") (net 4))
 (segment (start 40.75 41.65) (end 41.7 42.6) (width 1) (layer "F.Cu") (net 4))
 (segment (start 40.75 41.575) (end 40.05 42.275) (width 1) (layer "F.Cu") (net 4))
 (segment (start 33.55 38.805) (end 35.1 40.355) (width 1) (layer "F.Cu") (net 4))
 (segment (start 41.7 42.6) (end 45.2 42.6) (width 1) (layer "F.Cu") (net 4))
 (segment (start 40.75 40.85) (end 40.75 41.65) (width 1) (layer "F.Cu") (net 4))
 (segment (start 40.75 40.85) (end 40.75 41.575) (width 1) (layer "F.Cu") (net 4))
 (segment (start 45.525 42.275) (end 45.525 40.85) (width 1) (layer "F.Cu") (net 4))
 (segment (start 39.9 30.7) (end 38.4 32.2) (width 1) (layer "F.Cu") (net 4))
 (segment (start 38.4 36.7) (end 38.75 36.35) (width 1) (layer "F.Cu") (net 1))
 (segment (start 37.9 36.7) (end 38.4 36.7) (width 1) (layer "F.Cu") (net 1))
 (segment (start 44.3 30.7) (end 41.275 33.725) (width 1) (layer "F.Cu") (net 1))
 (segment (start 41.275 33.725) (end 37.9 33.725) (width 1) (layer "F.Cu") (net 1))
 (via (at 37.9 36.7) (size 0.8) (drill 0.4) (layers "F.Cu" "B.Cu") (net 1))
 (via (at 37.9 33.725) (size 0.8) (drill 0.4) (layers "F.Cu" "B.Cu") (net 1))
 (segment (start 37.9 33.725) (end 37.9 36.7) (width 1) (layer "B.Cu") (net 1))
 (segment (start 43.075 36.35) (end 40.825 36.35) (width 1) (layer "F.Cu") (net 2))
 (segment (start 40.825 38.575) (end 40.8 38.6) (width 1) (layer "F.Cu") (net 2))
 (segment (start 63.385 48.2) (end 64.935 49.75) (width 1) (layer "F.Cu") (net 2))
 (segment (start 51.96 49.75) (end 53.51 48.2) (width 1) (layer "F.Cu") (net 2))
 (segment (start 40.825 36.26207) (end 40.825 36.35) (width 1) (layer "F.Cu") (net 2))
 (segment (start 51.96 41.085) (end 46.175 35.3) (width 1) (layer "F.Cu") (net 2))
 (segment (start 35.1 35.275) (end 35.45 34.925) (width 1) (layer "F.Cu") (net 2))
 (segment (start 53.51 48.2) (end 63.385 48.2) (width 1) (layer "F.Cu") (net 2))
 (segment (start 35.45 34.925) (end 39.48793 34.925) (width 1) (layer "F.Cu") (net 2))
 (segment (start 46.175 35.3) (end 43.075 35.3) (width 1) (layer "F.Cu") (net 2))
 (segment (start 51.96 49.75) (end 51.96 41.085) (width 1) (layer "F.Cu") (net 2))
 (segment (start 39.48793 34.925) (end 40.825 36.26207) (width 1) (layer "F.Cu") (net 2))
 (segment (start 43.075 35.3) (end 43.075 36.35) (width 1) (layer "F.Cu") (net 2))
 (segment (start 40.825 36.35) (end 40.825 38.575) (width 1) (layer "F.Cu") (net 2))
 (segment (start 38.675 40.85) (end 38.15 40.85) (width 1) (layer "F.Cu") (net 3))
 (segment (start 38.725 38.6) (end 38.1 38.6) (width 1) (layer "F.Cu") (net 3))
 (segment (start 38.1 38.6) (end 37.9 38.8) (width 1) (layer "F.Cu") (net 3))
 (segment (start 38.15 40.85) (end 38.1 40.8) (width 1) (layer "F.Cu") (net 3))
 (via (at 37.9 38.8) (size 1) (drill 0.6) (layers "F.Cu" "B.Cu") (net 3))
 (via (at 38.1 40.8) (size 1) (drill 0.6) (layers "F.Cu" "B.Cu") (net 3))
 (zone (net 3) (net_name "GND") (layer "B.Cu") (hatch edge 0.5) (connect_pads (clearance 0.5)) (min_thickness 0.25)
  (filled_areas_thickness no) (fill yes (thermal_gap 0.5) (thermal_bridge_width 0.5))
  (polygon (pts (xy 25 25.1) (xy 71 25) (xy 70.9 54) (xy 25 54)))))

